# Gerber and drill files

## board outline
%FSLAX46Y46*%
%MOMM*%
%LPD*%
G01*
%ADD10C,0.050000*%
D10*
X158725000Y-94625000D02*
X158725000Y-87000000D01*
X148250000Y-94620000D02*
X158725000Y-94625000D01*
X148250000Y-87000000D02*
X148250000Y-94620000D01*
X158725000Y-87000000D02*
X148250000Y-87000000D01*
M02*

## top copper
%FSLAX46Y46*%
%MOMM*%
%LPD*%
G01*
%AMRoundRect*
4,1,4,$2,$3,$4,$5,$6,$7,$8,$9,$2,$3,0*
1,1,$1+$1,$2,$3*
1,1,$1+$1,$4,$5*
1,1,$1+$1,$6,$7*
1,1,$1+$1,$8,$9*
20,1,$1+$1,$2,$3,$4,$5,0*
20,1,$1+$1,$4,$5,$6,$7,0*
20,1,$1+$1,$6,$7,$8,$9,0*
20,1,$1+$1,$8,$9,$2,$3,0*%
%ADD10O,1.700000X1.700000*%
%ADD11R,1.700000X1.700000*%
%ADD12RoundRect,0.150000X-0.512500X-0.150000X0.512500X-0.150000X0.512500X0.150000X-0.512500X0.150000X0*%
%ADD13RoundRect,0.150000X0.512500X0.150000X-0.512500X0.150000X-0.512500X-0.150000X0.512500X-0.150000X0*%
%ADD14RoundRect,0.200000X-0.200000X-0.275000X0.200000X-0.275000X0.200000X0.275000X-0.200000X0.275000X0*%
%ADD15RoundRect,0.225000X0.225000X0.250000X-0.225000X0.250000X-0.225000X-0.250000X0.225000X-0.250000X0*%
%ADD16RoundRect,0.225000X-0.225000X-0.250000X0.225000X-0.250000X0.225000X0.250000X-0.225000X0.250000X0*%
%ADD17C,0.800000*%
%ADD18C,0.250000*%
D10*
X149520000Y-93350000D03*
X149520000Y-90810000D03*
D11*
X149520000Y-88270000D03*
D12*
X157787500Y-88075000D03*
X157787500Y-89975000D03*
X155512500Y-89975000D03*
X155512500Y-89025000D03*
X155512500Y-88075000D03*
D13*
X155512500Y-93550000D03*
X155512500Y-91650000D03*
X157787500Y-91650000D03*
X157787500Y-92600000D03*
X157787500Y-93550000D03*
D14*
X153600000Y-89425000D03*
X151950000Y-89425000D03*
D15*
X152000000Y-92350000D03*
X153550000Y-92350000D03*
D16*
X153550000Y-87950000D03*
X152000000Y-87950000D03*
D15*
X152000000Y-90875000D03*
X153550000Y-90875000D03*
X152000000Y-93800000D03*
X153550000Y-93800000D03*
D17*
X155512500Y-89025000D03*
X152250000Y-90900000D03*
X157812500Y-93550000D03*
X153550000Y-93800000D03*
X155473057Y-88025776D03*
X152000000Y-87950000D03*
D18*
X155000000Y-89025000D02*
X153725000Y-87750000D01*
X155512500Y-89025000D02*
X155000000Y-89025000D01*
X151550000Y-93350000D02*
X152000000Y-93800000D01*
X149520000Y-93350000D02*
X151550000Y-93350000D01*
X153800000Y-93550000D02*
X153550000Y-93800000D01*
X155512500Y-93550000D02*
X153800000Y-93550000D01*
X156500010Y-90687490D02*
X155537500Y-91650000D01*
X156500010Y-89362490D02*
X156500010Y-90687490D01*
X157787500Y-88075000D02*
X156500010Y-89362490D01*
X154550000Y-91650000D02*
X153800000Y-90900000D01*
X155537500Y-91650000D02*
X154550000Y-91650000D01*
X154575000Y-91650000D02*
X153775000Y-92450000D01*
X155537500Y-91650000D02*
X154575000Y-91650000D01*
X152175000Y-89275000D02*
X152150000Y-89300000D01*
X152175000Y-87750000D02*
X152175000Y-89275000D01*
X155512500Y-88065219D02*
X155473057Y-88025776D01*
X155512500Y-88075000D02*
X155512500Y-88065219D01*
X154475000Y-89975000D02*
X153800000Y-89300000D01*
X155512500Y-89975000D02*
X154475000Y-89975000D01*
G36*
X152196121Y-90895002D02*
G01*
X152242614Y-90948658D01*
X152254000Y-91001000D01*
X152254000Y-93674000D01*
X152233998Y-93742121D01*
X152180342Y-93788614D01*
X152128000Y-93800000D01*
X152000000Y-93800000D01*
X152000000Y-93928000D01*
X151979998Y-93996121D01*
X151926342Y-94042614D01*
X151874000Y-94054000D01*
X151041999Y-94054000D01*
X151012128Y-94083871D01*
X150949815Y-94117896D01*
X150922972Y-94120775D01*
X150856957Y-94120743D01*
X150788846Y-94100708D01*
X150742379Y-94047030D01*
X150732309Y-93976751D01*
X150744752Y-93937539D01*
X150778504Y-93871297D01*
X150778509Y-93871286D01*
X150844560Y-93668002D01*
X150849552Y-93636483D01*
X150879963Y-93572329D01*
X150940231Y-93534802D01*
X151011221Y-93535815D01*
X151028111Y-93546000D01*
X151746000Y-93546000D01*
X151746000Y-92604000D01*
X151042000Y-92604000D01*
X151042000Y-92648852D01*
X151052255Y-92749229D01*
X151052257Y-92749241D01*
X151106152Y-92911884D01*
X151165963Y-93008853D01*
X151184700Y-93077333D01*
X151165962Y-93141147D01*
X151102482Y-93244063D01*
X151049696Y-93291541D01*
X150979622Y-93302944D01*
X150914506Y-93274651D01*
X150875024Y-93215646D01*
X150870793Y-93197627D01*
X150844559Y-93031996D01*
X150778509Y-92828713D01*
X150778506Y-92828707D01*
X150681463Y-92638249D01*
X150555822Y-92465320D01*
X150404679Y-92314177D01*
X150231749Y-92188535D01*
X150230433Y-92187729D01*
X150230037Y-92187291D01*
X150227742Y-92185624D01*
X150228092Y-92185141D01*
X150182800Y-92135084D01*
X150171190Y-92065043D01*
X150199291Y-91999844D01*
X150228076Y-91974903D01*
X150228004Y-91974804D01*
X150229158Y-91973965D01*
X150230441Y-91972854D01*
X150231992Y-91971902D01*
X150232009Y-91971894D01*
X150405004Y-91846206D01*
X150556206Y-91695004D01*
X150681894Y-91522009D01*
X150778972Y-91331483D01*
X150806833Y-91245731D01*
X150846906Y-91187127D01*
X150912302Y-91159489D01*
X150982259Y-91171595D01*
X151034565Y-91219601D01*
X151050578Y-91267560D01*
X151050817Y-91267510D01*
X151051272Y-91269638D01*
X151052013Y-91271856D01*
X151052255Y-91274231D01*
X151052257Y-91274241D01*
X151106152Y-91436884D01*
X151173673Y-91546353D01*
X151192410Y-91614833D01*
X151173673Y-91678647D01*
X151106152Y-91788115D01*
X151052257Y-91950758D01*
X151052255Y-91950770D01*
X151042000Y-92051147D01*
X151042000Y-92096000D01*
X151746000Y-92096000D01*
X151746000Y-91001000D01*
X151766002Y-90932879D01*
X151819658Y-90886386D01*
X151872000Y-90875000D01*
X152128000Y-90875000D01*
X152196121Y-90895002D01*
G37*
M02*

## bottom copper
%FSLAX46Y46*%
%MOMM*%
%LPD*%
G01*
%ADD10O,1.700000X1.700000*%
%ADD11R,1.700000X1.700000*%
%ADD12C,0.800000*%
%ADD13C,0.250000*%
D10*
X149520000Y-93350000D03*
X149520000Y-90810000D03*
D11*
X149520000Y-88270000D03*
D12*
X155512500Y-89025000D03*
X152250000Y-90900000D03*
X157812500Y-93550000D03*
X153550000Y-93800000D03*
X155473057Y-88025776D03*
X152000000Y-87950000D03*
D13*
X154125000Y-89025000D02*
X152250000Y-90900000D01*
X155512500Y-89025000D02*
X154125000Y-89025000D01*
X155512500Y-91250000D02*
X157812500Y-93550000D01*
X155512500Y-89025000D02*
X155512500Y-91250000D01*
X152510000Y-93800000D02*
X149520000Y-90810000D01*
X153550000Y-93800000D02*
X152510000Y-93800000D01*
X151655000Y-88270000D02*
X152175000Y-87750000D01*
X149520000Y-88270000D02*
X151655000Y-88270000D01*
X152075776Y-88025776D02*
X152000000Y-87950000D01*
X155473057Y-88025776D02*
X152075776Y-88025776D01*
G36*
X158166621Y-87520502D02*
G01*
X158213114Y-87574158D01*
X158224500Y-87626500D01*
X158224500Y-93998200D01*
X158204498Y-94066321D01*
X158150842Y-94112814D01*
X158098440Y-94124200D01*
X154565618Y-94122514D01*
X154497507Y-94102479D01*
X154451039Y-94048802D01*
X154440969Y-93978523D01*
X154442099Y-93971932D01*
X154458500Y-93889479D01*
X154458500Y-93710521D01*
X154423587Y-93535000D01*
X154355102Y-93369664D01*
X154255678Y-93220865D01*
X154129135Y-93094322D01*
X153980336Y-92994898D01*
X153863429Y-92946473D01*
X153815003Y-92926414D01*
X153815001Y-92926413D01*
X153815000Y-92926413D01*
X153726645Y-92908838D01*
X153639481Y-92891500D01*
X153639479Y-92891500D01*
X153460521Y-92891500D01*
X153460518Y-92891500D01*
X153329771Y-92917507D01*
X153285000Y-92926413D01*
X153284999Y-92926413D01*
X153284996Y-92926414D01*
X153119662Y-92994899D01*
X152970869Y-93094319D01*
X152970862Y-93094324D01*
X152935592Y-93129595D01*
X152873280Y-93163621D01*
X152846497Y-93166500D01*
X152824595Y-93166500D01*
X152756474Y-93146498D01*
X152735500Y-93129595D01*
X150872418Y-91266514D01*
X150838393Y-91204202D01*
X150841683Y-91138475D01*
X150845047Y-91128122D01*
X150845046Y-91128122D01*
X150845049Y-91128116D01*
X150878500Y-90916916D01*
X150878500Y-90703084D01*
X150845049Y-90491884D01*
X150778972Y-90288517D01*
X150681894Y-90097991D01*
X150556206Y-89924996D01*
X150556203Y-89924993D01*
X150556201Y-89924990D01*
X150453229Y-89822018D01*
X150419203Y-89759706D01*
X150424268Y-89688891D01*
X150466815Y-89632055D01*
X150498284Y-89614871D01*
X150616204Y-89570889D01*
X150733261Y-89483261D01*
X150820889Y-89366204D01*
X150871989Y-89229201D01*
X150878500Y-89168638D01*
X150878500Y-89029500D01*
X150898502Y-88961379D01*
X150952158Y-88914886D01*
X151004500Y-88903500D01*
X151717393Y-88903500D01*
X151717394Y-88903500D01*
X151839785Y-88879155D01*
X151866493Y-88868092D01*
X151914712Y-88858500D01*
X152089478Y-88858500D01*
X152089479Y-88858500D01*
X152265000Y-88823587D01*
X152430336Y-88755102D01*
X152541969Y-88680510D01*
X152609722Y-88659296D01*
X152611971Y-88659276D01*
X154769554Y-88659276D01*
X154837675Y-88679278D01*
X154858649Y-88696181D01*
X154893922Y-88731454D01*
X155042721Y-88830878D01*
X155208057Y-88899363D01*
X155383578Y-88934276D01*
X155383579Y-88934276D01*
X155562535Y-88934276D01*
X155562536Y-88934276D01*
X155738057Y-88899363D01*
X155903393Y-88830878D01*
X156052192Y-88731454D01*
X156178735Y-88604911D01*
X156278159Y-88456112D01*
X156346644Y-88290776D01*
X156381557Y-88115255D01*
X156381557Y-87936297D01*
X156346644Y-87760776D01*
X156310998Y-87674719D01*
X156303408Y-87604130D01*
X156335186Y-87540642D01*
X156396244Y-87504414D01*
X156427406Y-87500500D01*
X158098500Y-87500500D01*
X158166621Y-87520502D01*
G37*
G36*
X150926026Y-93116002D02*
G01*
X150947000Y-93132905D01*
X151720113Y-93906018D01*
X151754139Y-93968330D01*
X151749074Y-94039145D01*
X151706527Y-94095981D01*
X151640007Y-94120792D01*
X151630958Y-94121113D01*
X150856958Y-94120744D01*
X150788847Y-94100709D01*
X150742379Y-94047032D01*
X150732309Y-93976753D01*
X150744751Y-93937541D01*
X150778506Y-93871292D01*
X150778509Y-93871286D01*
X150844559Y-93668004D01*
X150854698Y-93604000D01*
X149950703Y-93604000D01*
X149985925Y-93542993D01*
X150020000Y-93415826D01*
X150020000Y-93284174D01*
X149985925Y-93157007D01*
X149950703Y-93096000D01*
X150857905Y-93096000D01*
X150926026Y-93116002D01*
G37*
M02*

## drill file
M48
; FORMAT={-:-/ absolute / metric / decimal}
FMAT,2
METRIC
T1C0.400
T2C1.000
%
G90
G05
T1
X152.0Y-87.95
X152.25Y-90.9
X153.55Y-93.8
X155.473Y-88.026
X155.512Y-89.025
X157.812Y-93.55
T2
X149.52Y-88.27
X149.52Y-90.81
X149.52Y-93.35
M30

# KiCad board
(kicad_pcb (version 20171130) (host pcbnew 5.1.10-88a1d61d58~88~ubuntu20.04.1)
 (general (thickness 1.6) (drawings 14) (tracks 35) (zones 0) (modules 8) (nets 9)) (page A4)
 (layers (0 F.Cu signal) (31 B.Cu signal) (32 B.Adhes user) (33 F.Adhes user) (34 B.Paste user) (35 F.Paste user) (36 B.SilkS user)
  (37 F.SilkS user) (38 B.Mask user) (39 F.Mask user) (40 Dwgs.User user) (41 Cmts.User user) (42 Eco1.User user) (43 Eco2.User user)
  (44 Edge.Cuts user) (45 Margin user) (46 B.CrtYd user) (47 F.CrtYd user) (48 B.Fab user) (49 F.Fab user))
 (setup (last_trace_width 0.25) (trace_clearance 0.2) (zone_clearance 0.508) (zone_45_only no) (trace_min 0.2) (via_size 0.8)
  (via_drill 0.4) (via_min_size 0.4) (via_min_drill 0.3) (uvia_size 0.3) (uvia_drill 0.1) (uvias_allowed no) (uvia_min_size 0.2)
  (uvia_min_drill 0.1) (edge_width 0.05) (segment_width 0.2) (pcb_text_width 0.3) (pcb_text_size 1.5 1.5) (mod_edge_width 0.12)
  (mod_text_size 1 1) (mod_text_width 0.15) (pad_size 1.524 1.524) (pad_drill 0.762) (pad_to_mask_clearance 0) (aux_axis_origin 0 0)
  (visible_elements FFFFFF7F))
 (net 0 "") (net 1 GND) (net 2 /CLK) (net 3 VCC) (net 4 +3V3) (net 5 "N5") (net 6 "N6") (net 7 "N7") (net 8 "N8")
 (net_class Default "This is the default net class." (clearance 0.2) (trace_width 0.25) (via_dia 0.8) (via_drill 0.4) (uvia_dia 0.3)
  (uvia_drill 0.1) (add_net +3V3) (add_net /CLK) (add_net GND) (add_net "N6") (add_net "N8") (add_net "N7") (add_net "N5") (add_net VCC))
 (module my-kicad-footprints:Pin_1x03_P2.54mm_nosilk (layer F.Cu) (at 149.52 88.27)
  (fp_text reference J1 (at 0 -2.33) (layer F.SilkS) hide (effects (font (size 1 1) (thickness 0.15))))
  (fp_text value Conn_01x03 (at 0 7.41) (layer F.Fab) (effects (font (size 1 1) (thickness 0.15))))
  (pad 3 thru_hole oval (at 0 5.08) (size 1.7 1.7) (drill 1) (layers *.Cu *.Mask) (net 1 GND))
  (pad 2 thru_hole oval (at 0 2.54) (size 1.7 1.7) (drill 1) (layers *.Cu *.Mask) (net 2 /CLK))
  (pad 1 thru_hole rect (at 0 0) (size 1.7 1.7) (drill 1) (layers *.Cu *.Mask) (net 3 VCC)))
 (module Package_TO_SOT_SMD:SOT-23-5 (layer F.Cu) (at 156.65 89.025)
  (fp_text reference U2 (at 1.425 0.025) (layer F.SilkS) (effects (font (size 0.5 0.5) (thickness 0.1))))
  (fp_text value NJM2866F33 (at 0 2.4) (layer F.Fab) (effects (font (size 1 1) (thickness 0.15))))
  (pad 5 smd roundrect (at 1.1375 -0.95) (size 1.325 0.6) (layers F.Cu F.Paste F.Mask) (roundrect_rratio 0.25) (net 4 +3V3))
  (pad 4 smd roundrect (at 1.1375 0.95) (size 1.325 0.6) (layers F.Cu F.Paste F.Mask) (roundrect_rratio 0.25) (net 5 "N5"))
  (pad 3 smd roundrect (at -1.1375 0.95) (size 1.325 0.6) (layers F.Cu F.Paste F.Mask) (roundrect_rratio 0.25) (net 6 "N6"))
  (pad 2 smd roundrect (at -1.1375 0) (size 1.325 0.6) (layers F.Cu F.Paste F.Mask) (roundrect_rratio 0.25) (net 1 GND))
  (pad 1 smd roundrect (at -1.1375 -0.95) (size 1.325 0.6) (layers F.Cu F.Paste F.Mask) (roundrect_rratio 0.25) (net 3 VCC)))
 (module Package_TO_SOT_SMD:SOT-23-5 (layer F.Cu) (at 156.65 92.6 180)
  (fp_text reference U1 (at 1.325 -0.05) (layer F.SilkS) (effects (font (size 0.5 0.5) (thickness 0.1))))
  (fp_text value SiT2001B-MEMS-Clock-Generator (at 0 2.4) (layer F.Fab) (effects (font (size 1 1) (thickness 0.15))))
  (pad 5 smd roundrect (at 1.1375 -0.95 180) (size 1.325 0.6) (layers F.Cu F.Paste F.Mask) (roundrect_rratio 0.25) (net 2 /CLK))
  (pad 4 smd roundrect (at 1.1375 0.95 180) (size 1.325 0.6) (layers F.Cu F.Paste F.Mask) (roundrect_rratio 0.25) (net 4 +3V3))
  (pad 3 smd roundrect (at -1.1375 0.95 180) (size 1.325 0.6) (layers F.Cu F.Paste F.Mask) (roundrect_rratio 0.25) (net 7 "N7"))
  (pad 2 smd roundrect (at -1.1375 0 180) (size 1.325 0.6) (layers F.Cu F.Paste F.Mask) (roundrect_rratio 0.25) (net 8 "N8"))
  (pad 1 smd roundrect (at -1.1375 -0.95 180) (size 1.325 0.6) (layers F.Cu F.Paste F.Mask) (roundrect_rratio 0.25) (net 1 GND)))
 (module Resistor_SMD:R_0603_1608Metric (layer F.Cu) (at 152.775 89.425)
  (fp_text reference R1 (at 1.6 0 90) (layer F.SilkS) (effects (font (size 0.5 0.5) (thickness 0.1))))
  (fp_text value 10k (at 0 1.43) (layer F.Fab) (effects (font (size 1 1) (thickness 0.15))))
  (pad 2 smd roundrect (at 0.825 0) (size 0.8 0.95) (layers F.Cu F.Paste F.Mask) (roundrect_rratio 0.25) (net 6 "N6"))
  (pad 1 smd roundrect (at -0.825 0) (size 0.8 0.95) (layers F.Cu F.Paste F.Mask) (roundrect_rratio 0.25) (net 3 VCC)))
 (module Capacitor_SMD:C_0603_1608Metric (layer F.Cu) (at 152.775 92.35 180)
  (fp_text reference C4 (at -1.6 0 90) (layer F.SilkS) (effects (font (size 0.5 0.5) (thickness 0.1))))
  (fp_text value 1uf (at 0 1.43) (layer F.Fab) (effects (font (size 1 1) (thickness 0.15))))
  (pad 2 smd roundrect (at 0.775 0 180) (size 0.9 0.95) (layers F.Cu F.Paste F.Mask) (roundrect_rratio 0.25) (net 1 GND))
  (pad 1 smd roundrect (at -0.775 0 180) (size 0.9 0.95) (layers F.Cu F.Paste F.Mask) (roundrect_rratio 0.25) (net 4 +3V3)))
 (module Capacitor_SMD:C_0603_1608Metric (layer F.Cu) (at 152.775 87.95)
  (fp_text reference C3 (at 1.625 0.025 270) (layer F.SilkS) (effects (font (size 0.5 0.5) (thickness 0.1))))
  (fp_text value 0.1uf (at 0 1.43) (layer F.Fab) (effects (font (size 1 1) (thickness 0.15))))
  (pad 2 smd roundrect (at 0.775 0) (size 0.9 0.95) (layers F.Cu F.Paste F.Mask) (roundrect_rratio 0.25) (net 1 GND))
  (pad 1 smd roundrect (at -0.775 0) (size 0.9 0.95) (layers F.Cu F.Paste F.Mask) (roundrect_rratio 0.25) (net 3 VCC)))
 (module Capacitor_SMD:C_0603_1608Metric (layer F.Cu) (at 152.775 90.875 180)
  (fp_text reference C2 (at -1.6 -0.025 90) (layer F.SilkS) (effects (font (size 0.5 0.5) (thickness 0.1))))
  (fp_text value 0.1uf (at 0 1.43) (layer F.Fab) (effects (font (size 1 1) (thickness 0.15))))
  (pad 2 smd roundrect (at 0.775 0 180) (size 0.9 0.95) (layers F.Cu F.Paste F.Mask) (roundrect_rratio 0.25) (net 1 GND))
  (pad 1 smd roundrect (at -0.775 0 180) (size 0.9 0.95) (layers F.Cu F.Paste F.Mask) (roundrect_rratio 0.25) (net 4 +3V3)))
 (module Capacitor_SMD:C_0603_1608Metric (layer F.Cu) (at 152.775 93.8 180)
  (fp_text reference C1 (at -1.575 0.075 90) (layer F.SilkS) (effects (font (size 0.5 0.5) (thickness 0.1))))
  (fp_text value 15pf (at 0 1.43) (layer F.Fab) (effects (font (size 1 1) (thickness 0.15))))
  (pad 2 smd roundrect (at 0.775 0 180) (size 0.9 0.95) (layers F.Cu F.Paste F.Mask) (roundrect_rratio 0.25) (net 1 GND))
  (pad 1 smd roundrect (at -0.775 0 180) (size 0.9 0.95) (layers F.Cu F.Paste F.Mask) (roundrect_rratio 0.25) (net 2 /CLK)))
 (gr_line (start 158.725 94.625) (end 158.725 87) (layer Edge.Cuts) (width 0.05))
 (gr_line (start 148.25 94.62) (end 158.725 94.625) (layer Edge.Cuts) (width 0.05))
 (gr_line (start 148.25 87) (end 148.25 94.62) (layer Edge.Cuts) (width 0.05))
 (gr_line (start 158.725 87) (end 148.25 87) (layer Edge.Cuts) (width 0.05))
 (segment (start 155 89.025) (end 153.725 87.75) (width 0.25) (layer F.Cu) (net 1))
 (segment (start 155.5125 89.025) (end 155 89.025) (width 0.25) (layer F.Cu) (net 1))
 (via (at 155.5125 89.025) (size 0.8) (drill 0.4) (layers F.Cu B.Cu) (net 1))
 (via (at 152.25 90.9) (size 0.8) (drill 0.4) (layers F.Cu B.Cu) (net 1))
 (segment (start 154.125 89.025) (end 152.25 90.9) (width 0.25) (layer B.Cu) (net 1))
 (segment (start 155.5125 89.025) (end 154.125 89.025) (width 0.25) (layer B.Cu) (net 1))
 (via (at 157.8125 93.55) (size 0.8) (drill 0.4) (layers F.Cu B.Cu) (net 1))
 (segment (start 155.5125 91.25) (end 157.8125 93.55) (width 0.25) (layer B.Cu) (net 1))
 (segment (start 155.5125 89.025) (end 155.5125 91.25) (width 0.25) (layer B.Cu) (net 1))
 (segment (start 151.55 93.35) (end 152 93.8) (width 0.25) (layer F.Cu) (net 1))
 (segment (start 149.52 93.35) (end 151.55 93.35) (width 0.25) (layer F.Cu) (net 1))
 (via (at 153.55 93.8) (size 0.8) (drill 0.4) (layers F.Cu B.Cu) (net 2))
 (segment (start 153.8 93.55) (end 153.55 93.8) (width 0.25) (layer F.Cu) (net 2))
 (segment (start 155.5125 93.55) (end 153.8 93.55) (width 0.25) (layer F.Cu) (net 2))
 (segment (start 152.51 93.8) (end 149.52 90.81) (width 0.25) (layer B.Cu) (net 2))
 (segment (start 153.55 93.8) (end 152.51 93.8) (width 0.25) (layer B.Cu) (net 2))
 (segment (start 156.50001 90.68749) (end 155.5375 91.65) (width 0.25) (layer F.Cu) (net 4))
 (segment (start 156.50001 89.36249) (end 156.50001 90.68749) (width 0.25) (layer F.Cu) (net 4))
 (segment (start 157.7875 88.075) (end 156.50001 89.36249) (width 0.25) (layer F.Cu) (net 4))
 (segment (start 154.55 91.65) (end 153.8 90.9) (width 0.25) (layer F.Cu) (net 4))
 (segment (start 155.5375 91.65) (end 154.55 91.65) (width 0.25) (layer F.Cu) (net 4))
 (segment (start 154.575 91.65) (end 153.775 92.45) (width 0.25) (layer F.Cu) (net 4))
 (segment (start 155.5375 91.65) (end 154.575 91.65) (width 0.25) (layer F.Cu) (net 4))
 (segment (start 151.655 88.27) (end 152.175 87.75) (width 0.25) (layer B.Cu) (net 3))
 (segment (start 149.52 88.27) (end 151.655 88.27) (width 0.25) (layer B.Cu) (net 3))
 (segment (start 152.175 89.275) (end 152.15 89.3) (width 0.25) (layer F.Cu) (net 3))
 (segment (start 152.175 87.75) (end 152.175 89.275) (width 0.25) (layer F.Cu) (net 3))
 (via (at 155.473057 88.025776) (size 0.8) (drill 0.4) (layers F.Cu B.Cu) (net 3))
 (segment (start 155.5125 88.065219) (end 155.473057 88.025776) (width 0.25) (layer F.Cu) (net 3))
 (segment (start 155.5125 88.075) (end 155.5125 88.065219) (width 0.25) (layer F.Cu) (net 3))
 (via (at 152 87.95) (size 0.8) (drill 0.4) (layers F.Cu B.Cu) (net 3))
 (segment (start 152.075776 88.025776) (end 152 87.95) (width 0.25) (layer B.Cu) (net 3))
 (segment (start 155.473057 88.025776) (end 152.075776 88.025776) (width 0.25) (layer B.Cu) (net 3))
 (segment (start 154.475 89.975) (end 153.8 89.3) (width 0.25) (layer F.Cu) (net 6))
 (segment (start 155.5125 89.975) (end 154.475 89.975) (width 0.25) (layer F.Cu) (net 6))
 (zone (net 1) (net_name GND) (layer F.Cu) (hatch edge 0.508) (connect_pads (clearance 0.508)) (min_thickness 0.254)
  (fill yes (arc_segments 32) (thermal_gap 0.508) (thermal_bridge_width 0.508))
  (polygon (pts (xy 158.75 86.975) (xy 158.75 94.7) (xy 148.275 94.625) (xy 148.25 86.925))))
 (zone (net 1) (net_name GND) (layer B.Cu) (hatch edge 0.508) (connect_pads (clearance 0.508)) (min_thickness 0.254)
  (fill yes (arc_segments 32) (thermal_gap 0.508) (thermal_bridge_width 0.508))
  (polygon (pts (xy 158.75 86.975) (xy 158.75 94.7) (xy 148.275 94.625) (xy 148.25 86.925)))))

